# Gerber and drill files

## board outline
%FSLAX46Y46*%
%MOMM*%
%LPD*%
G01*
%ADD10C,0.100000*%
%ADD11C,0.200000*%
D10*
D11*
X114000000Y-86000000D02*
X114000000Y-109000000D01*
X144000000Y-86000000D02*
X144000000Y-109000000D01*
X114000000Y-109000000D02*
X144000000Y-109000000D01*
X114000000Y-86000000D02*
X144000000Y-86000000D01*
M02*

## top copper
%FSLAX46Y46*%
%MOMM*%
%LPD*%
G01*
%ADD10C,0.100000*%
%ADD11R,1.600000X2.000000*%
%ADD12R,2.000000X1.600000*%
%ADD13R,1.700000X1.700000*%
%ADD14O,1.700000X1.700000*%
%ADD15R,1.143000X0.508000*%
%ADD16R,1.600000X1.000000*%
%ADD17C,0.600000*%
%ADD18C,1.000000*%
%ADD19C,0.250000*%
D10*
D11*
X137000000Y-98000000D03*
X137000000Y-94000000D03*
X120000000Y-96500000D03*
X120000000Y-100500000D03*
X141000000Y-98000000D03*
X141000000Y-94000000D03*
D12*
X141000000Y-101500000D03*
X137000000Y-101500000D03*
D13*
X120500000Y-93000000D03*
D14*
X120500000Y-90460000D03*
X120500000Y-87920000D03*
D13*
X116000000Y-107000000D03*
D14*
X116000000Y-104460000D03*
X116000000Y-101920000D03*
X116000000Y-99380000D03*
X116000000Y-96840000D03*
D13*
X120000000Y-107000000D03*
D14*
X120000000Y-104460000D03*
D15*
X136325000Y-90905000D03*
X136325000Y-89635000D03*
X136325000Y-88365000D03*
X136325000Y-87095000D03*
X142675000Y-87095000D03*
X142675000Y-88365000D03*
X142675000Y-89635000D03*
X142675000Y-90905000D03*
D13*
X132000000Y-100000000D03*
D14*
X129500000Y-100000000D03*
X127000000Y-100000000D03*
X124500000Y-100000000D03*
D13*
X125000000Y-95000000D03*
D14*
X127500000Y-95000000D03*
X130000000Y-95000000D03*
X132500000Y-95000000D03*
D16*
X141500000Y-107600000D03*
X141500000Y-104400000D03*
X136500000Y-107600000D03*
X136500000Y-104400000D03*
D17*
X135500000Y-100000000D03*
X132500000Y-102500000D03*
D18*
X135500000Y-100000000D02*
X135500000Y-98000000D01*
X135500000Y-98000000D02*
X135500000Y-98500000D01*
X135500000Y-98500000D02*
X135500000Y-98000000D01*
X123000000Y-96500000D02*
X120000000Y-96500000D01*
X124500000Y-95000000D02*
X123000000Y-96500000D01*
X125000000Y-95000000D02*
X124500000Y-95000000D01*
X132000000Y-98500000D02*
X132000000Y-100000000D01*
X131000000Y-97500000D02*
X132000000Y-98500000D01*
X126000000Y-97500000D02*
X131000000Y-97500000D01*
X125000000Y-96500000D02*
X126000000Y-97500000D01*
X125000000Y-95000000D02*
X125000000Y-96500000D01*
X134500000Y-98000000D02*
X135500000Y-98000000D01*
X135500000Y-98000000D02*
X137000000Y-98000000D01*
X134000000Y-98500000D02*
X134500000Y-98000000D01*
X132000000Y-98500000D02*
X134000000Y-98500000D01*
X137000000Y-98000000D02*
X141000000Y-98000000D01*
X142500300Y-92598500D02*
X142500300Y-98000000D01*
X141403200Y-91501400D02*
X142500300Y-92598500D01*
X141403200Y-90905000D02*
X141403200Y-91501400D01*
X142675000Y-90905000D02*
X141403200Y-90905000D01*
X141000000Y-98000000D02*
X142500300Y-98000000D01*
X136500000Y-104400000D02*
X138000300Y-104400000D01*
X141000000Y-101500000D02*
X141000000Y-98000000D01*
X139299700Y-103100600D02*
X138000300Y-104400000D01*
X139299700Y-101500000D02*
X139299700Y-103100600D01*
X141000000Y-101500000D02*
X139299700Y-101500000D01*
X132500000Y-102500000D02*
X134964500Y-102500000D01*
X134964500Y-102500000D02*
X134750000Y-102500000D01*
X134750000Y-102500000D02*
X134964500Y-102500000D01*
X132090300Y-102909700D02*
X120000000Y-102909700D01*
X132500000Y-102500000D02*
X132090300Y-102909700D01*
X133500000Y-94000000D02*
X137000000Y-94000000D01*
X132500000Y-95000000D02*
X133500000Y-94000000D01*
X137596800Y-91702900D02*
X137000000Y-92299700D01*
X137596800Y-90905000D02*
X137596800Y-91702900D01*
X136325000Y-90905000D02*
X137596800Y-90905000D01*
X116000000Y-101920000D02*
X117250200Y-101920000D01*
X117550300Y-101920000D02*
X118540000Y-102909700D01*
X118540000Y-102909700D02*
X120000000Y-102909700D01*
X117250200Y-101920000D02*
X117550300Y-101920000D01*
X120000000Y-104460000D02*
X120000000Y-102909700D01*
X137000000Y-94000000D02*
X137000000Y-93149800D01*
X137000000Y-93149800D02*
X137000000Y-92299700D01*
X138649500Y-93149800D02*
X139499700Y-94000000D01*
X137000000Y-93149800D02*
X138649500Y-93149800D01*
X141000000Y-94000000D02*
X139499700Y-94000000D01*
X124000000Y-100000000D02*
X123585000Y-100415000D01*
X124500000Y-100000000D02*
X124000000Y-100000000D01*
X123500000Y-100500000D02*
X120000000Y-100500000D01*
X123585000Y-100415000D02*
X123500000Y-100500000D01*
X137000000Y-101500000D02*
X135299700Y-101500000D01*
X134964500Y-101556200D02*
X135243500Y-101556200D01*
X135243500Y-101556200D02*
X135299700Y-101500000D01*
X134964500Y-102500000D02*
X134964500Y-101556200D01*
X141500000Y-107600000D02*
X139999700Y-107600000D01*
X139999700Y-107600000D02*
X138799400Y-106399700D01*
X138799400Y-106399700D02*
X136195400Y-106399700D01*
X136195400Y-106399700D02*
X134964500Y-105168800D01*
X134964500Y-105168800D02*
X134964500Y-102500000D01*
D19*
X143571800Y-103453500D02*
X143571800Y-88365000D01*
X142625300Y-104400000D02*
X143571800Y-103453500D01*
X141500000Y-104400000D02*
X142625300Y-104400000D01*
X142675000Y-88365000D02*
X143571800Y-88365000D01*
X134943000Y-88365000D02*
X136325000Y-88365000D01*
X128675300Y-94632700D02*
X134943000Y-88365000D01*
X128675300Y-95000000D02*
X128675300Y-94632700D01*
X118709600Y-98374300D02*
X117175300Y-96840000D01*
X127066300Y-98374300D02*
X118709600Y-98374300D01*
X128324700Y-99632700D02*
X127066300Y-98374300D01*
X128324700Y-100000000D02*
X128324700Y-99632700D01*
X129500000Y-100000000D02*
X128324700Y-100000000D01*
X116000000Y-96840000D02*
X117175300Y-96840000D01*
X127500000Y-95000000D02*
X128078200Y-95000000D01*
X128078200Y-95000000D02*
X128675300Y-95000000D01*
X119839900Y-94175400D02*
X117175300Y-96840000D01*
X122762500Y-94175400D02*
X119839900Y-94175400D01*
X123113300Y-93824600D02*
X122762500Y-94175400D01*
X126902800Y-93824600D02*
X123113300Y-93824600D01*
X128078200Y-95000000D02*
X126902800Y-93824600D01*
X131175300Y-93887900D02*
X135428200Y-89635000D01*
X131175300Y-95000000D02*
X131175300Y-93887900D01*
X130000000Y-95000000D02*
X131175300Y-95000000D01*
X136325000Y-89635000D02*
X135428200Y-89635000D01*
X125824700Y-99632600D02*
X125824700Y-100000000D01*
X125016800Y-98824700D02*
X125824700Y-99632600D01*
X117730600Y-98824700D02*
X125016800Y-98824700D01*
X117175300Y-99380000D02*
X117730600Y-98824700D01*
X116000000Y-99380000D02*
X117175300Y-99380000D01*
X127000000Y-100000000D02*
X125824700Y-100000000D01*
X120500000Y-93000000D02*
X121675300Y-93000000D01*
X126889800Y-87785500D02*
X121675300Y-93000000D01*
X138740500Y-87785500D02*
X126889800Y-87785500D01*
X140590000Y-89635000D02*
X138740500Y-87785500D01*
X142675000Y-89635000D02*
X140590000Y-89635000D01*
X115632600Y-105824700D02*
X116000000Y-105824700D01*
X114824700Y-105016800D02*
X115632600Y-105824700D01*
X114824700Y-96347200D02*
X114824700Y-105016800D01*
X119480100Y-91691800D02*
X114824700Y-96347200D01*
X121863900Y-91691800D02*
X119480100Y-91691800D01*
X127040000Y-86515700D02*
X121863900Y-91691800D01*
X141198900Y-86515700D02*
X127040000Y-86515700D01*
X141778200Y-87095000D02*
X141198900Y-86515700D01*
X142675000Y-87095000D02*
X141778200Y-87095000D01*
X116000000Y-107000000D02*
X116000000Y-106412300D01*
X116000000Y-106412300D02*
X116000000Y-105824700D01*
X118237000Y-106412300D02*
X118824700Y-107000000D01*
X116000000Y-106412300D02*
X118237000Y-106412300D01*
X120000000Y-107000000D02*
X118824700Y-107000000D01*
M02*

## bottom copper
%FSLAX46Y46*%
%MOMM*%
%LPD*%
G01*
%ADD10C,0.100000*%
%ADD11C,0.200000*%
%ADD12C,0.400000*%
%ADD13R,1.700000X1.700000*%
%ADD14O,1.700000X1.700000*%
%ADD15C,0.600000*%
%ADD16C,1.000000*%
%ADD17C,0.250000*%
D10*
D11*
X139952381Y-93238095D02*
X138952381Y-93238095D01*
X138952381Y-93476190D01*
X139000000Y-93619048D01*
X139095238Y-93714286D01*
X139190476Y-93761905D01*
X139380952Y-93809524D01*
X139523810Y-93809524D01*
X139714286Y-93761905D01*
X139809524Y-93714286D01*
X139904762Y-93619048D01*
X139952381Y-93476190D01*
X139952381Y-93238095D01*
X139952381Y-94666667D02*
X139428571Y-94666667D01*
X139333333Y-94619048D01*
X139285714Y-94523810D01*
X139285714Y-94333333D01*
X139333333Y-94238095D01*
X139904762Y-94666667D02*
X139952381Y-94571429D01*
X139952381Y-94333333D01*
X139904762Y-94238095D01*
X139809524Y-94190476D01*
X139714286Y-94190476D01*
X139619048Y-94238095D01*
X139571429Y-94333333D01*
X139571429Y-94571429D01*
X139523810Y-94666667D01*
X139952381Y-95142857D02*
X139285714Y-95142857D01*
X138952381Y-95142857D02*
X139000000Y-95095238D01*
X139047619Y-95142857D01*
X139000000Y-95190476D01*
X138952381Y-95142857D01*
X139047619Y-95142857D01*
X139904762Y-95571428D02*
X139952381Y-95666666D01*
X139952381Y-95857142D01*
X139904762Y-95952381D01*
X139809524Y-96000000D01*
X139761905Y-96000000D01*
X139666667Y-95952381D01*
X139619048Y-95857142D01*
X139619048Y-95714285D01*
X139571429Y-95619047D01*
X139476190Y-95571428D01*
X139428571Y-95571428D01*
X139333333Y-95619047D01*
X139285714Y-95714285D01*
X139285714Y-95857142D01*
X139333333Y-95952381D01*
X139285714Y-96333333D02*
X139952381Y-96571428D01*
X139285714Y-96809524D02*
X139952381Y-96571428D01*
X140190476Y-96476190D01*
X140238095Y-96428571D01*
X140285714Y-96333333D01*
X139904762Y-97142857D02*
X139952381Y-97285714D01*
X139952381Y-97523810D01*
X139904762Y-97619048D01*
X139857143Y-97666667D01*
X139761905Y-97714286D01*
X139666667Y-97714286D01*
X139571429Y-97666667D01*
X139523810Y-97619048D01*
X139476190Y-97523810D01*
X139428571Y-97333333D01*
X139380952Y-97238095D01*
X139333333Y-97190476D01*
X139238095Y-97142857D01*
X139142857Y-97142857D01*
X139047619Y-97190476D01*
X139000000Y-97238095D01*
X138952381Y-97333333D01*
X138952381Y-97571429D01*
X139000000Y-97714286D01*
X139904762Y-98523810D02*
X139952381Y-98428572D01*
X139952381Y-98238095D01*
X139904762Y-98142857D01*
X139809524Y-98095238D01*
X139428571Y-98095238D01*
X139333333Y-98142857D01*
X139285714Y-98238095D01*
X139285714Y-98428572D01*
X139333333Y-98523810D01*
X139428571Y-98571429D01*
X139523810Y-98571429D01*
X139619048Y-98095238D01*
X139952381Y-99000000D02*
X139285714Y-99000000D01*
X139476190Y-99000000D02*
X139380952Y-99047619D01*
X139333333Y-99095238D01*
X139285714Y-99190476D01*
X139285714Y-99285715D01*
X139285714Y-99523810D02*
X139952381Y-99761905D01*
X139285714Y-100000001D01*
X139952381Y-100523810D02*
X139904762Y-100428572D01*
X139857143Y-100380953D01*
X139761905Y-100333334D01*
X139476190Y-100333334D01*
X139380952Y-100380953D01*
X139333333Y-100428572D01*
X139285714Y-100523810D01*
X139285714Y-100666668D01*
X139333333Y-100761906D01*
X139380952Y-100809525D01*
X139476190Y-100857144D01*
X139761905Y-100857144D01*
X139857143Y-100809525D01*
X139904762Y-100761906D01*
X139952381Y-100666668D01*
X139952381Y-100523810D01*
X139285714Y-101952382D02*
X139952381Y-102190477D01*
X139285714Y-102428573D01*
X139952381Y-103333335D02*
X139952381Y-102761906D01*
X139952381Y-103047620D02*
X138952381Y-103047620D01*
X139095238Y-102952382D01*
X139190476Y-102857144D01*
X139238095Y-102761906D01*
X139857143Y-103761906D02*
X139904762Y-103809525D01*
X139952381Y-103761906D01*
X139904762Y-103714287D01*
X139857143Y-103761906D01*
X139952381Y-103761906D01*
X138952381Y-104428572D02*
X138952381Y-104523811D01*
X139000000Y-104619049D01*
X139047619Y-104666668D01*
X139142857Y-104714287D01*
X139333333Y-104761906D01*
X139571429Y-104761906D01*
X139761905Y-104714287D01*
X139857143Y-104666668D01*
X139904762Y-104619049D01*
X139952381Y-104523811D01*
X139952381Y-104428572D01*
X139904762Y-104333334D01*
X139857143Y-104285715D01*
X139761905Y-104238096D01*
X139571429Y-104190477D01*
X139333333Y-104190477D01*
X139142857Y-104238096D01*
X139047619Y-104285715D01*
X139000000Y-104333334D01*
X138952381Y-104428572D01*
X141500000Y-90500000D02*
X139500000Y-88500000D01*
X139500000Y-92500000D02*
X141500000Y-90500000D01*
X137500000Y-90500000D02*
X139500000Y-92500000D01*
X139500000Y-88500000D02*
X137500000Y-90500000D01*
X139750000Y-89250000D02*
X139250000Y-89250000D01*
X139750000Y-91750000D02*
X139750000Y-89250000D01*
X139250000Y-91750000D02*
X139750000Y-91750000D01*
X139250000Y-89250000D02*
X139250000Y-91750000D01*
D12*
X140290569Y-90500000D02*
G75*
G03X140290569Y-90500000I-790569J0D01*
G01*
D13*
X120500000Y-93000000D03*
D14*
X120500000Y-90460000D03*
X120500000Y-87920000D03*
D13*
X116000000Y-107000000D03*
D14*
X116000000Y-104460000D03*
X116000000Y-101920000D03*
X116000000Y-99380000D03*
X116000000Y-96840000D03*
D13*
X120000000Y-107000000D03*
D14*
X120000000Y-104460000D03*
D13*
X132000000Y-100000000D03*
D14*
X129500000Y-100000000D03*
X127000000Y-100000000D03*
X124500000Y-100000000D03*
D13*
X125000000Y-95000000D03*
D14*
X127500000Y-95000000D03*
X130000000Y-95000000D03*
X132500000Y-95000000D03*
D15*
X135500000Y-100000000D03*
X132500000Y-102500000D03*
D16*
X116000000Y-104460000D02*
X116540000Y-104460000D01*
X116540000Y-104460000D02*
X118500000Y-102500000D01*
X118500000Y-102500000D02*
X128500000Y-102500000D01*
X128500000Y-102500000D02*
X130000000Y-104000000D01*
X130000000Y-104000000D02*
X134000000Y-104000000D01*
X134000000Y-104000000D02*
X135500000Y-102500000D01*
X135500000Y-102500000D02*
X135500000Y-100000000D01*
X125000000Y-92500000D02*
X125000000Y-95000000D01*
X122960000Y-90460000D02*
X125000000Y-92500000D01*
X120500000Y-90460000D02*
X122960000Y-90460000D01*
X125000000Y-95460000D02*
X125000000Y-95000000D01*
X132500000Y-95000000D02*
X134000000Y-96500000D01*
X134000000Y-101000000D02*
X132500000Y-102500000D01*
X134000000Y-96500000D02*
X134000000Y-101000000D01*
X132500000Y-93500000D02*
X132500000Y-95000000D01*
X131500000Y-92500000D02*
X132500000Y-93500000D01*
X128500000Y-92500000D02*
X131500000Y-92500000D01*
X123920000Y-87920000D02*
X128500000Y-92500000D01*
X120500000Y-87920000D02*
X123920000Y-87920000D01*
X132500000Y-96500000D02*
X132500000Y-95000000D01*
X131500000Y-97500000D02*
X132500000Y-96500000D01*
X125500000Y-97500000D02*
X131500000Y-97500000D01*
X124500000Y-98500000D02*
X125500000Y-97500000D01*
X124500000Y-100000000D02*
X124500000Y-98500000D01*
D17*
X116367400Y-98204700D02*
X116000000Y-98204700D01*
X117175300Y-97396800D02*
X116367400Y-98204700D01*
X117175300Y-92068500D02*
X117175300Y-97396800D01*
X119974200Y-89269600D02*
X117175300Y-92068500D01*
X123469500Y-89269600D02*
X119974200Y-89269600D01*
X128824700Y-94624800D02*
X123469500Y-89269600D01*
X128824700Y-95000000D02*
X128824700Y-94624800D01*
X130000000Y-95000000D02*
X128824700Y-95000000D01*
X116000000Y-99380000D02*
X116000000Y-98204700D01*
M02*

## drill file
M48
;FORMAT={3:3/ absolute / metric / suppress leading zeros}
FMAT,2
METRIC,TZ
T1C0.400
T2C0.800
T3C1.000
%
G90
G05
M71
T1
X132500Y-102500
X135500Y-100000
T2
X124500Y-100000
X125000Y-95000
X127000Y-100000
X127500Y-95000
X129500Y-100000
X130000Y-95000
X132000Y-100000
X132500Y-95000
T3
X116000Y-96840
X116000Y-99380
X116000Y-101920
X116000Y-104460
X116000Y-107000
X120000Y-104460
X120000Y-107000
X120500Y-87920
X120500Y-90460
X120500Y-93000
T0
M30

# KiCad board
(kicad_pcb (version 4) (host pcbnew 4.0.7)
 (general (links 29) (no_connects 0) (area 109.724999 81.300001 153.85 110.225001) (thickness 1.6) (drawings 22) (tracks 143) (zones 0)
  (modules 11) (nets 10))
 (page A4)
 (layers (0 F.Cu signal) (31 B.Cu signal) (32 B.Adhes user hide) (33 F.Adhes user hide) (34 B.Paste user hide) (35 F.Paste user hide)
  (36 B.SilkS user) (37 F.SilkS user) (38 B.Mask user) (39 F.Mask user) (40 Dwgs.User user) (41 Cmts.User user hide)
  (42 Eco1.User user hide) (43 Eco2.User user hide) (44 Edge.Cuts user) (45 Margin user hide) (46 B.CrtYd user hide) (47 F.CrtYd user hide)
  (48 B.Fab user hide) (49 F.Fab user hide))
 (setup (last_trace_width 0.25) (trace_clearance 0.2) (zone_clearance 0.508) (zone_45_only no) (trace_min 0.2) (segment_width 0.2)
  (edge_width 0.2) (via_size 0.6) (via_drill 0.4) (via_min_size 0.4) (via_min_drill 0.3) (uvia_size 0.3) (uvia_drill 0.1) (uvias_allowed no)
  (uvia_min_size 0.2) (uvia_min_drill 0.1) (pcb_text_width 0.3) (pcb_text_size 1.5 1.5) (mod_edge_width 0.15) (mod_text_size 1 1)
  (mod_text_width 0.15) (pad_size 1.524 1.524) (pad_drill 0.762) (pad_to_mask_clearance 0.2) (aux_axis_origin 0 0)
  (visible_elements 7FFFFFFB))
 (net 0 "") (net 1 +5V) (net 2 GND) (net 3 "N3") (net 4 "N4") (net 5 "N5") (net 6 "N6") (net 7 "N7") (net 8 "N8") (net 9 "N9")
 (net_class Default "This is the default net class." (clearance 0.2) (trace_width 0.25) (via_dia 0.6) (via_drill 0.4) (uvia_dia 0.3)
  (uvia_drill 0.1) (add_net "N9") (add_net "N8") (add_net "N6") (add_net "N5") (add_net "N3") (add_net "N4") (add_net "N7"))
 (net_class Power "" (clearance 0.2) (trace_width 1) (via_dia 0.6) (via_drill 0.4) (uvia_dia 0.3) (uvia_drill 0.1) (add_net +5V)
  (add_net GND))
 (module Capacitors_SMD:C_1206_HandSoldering (layer F.Cu) (at 137 96 90)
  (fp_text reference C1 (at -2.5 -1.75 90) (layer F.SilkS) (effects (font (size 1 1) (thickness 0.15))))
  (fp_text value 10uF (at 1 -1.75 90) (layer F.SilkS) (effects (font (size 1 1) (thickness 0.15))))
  (pad 1 smd rect (at -2 0 90) (size 2 1.6) (layers F.Cu F.Paste F.Mask) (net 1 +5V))
  (pad 2 smd rect (at 2 0 90) (size 2 1.6) (layers F.Cu F.Paste F.Mask) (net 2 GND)))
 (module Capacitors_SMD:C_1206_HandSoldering (layer F.Cu) (at 120 98.5 270)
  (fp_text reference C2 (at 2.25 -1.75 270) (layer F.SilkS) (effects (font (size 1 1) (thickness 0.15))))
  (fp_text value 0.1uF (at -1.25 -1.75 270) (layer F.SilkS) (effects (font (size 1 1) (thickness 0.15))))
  (pad 1 smd rect (at -2 0 270) (size 2 1.6) (layers F.Cu F.Paste F.Mask) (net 1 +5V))
  (pad 2 smd rect (at 2 0 270) (size 2 1.6) (layers F.Cu F.Paste F.Mask) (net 2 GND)))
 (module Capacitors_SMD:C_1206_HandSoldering (layer F.Cu) (at 141 96 90)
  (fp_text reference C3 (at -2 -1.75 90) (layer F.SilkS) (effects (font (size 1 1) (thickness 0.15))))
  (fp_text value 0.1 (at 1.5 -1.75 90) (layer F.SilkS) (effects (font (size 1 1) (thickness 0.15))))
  (pad 1 smd rect (at -2 0 90) (size 2 1.6) (layers F.Cu F.Paste F.Mask) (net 1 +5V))
  (pad 2 smd rect (at 2 0 90) (size 2 1.6) (layers F.Cu F.Paste F.Mask) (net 2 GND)))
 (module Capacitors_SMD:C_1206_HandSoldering (layer F.Cu) (at 139 101.5 180)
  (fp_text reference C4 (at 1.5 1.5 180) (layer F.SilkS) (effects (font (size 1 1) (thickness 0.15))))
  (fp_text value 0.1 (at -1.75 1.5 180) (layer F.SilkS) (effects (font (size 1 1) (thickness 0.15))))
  (pad 1 smd rect (at -2 0 180) (size 2 1.6) (layers F.Cu F.Paste F.Mask) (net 1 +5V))
  (pad 2 smd rect (at 2 0 180) (size 2 1.6) (layers F.Cu F.Paste F.Mask) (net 2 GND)))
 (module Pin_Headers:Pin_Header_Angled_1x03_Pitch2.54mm (layer F.Cu) (at 120.5 93 180)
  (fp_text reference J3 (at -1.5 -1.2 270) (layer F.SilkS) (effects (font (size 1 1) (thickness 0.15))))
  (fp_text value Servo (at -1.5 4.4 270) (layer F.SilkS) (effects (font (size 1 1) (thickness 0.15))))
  (pad 1 thru_hole rect (at 0 0 180) (size 1.7 1.7) (drill 1) (layers *.Cu *.Mask) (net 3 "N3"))
  (pad 2 thru_hole oval (at 0 2.54 180) (size 1.7 1.7) (drill 1) (layers *.Cu *.Mask) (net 1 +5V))
  (pad 3 thru_hole oval (at 0 5.08 180) (size 1.7 1.7) (drill 1) (layers *.Cu *.Mask) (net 2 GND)))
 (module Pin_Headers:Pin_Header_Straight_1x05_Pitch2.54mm (layer F.Cu) (at 116 107 180)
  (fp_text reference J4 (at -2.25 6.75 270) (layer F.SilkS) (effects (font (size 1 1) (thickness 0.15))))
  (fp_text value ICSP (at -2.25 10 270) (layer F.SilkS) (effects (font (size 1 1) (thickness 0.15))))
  (pad 1 thru_hole rect (at 0 0 180) (size 1.7 1.7) (drill 1) (layers *.Cu *.Mask) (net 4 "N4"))
  (pad 2 thru_hole oval (at 0 2.54 180) (size 1.7 1.7) (drill 1) (layers *.Cu *.Mask) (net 1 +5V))
  (pad 3 thru_hole oval (at 0 5.08 180) (size 1.7 1.7) (drill 1) (layers *.Cu *.Mask) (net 2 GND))
  (pad 4 thru_hole oval (at 0 7.62 180) (size 1.7 1.7) (drill 1) (layers *.Cu *.Mask) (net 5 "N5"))
  (pad 5 thru_hole oval (at 0 10.16 180) (size 1.7 1.7) (drill 1) (layers *.Cu *.Mask) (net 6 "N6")))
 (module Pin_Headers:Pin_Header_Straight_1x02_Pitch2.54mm (layer F.Cu) (at 120 107 180)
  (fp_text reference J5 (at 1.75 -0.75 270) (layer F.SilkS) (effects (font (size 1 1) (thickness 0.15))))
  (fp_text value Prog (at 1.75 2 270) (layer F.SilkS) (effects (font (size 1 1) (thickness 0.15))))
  (pad 1 thru_hole rect (at 0 0 180) (size 1.7 1.7) (drill 1) (layers *.Cu *.Mask) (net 4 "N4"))
  (pad 2 thru_hole oval (at 0 2.54 180) (size 1.7 1.7) (drill 1) (layers *.Cu *.Mask) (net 2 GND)))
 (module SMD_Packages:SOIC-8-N (layer F.Cu) (at 139.5 89 90)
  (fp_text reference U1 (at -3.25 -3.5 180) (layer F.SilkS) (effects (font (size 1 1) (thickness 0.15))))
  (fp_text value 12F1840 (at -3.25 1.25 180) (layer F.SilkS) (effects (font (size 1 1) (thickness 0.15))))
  (pad 8 smd rect (at -1.905 -3.175 90) (size 0.508 1.143) (layers F.Cu F.Paste F.Mask) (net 2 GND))
  (pad 7 smd rect (at -0.635 -3.175 90) (size 0.508 1.143) (layers F.Cu F.Paste F.Mask) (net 5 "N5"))
  (pad 6 smd rect (at 0.635 -3.175 90) (size 0.508 1.143) (layers F.Cu F.Paste F.Mask) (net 6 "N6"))
  (pad 5 smd rect (at 1.905 -3.175 90) (size 0.508 1.143) (layers F.Cu F.Paste F.Mask) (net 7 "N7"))
  (pad 4 smd rect (at 1.905 3.175 90) (size 0.508 1.143) (layers F.Cu F.Paste F.Mask) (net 4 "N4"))
  (pad 3 smd rect (at 0.635 3.175 90) (size 0.508 1.143) (layers F.Cu F.Paste F.Mask) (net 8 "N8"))
  (pad 2 smd rect (at -0.635 3.175 90) (size 0.508 1.143) (layers F.Cu F.Paste F.Mask) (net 3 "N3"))
  (pad 1 smd rect (at -1.905 3.175 90) (size 0.508 1.143) (layers F.Cu F.Paste F.Mask) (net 1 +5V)))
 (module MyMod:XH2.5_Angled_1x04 (layer F.Cu) (at 132 100 270)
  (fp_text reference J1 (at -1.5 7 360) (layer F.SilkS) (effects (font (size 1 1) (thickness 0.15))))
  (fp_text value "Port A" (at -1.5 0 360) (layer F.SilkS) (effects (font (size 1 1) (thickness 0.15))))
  (pad 1 thru_hole rect (at 0 0 270) (size 1.7 1.7) (drill 0.8) (layers *.Cu *.Mask) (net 1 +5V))
  (pad 2 thru_hole oval (at 0 2.5 270) (size 1.7 1.7) (drill 0.8) (layers *.Cu *.Mask) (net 6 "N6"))
  (pad 3 thru_hole oval (at 0 5 270) (size 1.7 1.7) (drill 0.8) (layers *.Cu *.Mask) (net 5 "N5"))
  (pad 4 thru_hole oval (at 0 7.5 270) (size 1.7 1.7) (drill 0.8) (layers *.Cu *.Mask) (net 2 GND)))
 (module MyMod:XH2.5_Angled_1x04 (layer F.Cu) (at 125 95 90)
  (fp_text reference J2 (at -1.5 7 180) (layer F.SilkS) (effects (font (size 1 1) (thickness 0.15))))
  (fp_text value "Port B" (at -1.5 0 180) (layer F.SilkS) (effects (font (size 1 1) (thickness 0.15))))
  (pad 1 thru_hole rect (at 0 0 90) (size 1.7 1.7) (drill 0.8) (layers *.Cu *.Mask) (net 1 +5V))
  (pad 2 thru_hole oval (at 0 2.5 90) (size 1.7 1.7) (drill 0.8) (layers *.Cu *.Mask) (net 6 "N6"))
  (pad 3 thru_hole oval (at 0 5 90) (size 1.7 1.7) (drill 0.8) (layers *.Cu *.Mask) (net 5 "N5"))
  (pad 4 thru_hole oval (at 0 7.5 90) (size 1.7 1.7) (drill 0.8) (layers *.Cu *.Mask) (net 2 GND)))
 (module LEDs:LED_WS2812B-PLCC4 (layer F.Cu) (at 139 106)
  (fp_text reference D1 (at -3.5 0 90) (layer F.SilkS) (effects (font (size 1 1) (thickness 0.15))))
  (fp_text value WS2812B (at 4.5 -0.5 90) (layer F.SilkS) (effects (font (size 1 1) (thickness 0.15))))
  (pad 3 smd rect (at 2.5 1.6) (size 1.6 1) (layers F.Cu F.Paste F.Mask) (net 2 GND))
  (pad 4 smd rect (at 2.5 -1.6) (size 1.6 1) (layers F.Cu F.Paste F.Mask) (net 8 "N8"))
  (pad 2 smd rect (at -2.5 1.6) (size 1.6 1) (layers F.Cu F.Paste F.Mask) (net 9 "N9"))
  (pad 1 smd rect (at -2.5 -1.6) (size 1.6 1) (layers F.Cu F.Paste F.Mask) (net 1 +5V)))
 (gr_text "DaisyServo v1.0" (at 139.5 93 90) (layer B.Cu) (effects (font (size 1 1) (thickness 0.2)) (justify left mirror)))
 (gr_line (start 141.5 90.5) (end 139.5 88.5) (angle 90) (layer B.Cu) (width 0.2))
 (gr_line (start 139.5 92.5) (end 141.5 90.5) (angle 90) (layer B.Cu) (width 0.2))
 (gr_line (start 137.5 90.5) (end 139.5 92.5) (angle 90) (layer B.Cu) (width 0.2))
 (gr_line (start 139.5 88.5) (end 137.5 90.5) (angle 90) (layer B.Cu) (width 0.2))
 (gr_line (start 139.75 89.25) (end 139.25 89.25) (angle 90) (layer B.Cu) (width 0.2))
 (gr_line (start 139.75 91.75) (end 139.75 89.25) (angle 90) (layer B.Cu) (width 0.2))
 (gr_line (start 139.25 91.75) (end 139.75 91.75) (angle 90) (layer B.Cu) (width 0.2))
 (gr_line (start 139.25 89.25) (end 139.25 91.75) (angle 90) (layer B.Cu) (width 0.2))
 (gr_circle (center 139.5 90.5) (end 139.75 89.75) (layer B.Cu) (width 0.4))
 (gr_line (start 114 86) (end 114 109) (angle 90) (layer Edge.Cuts) (width 0.2))
 (gr_line (start 144 86) (end 144 109) (angle 90) (layer Edge.Cuts) (width 0.2))
 (gr_line (start 114 109) (end 144 109) (angle 90) (layer Edge.Cuts) (width 0.2))
 (gr_line (start 114 86) (end 144 86) (angle 90) (layer Edge.Cuts) (width 0.2))
 (segment (start 116 104.46) (end 116.54 104.46) (width 1) (layer B.Cu) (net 1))
 (segment (start 116.54 104.46) (end 118.5 102.5) (width 1) (layer B.Cu) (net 1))
 (segment (start 118.5 102.5) (end 128.5 102.5) (width 1) (layer B.Cu) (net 1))
 (segment (start 128.5 102.5) (end 130 104) (width 1) (layer B.Cu) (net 1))
 (segment (start 130 104) (end 134 104) (width 1) (layer B.Cu) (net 1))
 (segment (start 134 104) (end 135.5 102.5) (width 1) (layer B.Cu) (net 1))
 (segment (start 135.5 102.5) (end 135.5 100) (width 1) (layer B.Cu) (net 1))
 (via (at 135.5 100) (size 0.6) (drill 0.4) (layers F.Cu B.Cu) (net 1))
 (segment (start 135.5 100) (end 135.5 98) (width 1) (layer F.Cu) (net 1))
 (segment (start 135.5 98) (end 135.5 98.5) (width 1) (layer F.Cu) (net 1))
 (segment (start 135.5 98.5) (end 135.5 98) (width 1) (layer F.Cu) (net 1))
 (segment (start 123 96.5) (end 120 96.5) (width 1) (layer F.Cu) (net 1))
 (segment (start 124.5 95) (end 123 96.5) (width 1) (layer F.Cu) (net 1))
 (segment (start 125 95) (end 124.5 95) (width 1) (layer F.Cu) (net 1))
 (segment (start 125 92.5) (end 125 95) (width 1) (layer B.Cu) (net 1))
 (segment (start 122.96 90.46) (end 125 92.5) (width 1) (layer B.Cu) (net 1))
 (segment (start 120.5 90.46) (end 122.96 90.46) (width 1) (layer B.Cu) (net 1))
 (segment (start 132 98.5) (end 132 100) (width 1) (layer F.Cu) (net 1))
 (segment (start 131 97.5) (end 132 98.5) (width 1) (layer F.Cu) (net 1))
 (segment (start 126 97.5) (end 131 97.5) (width 1) (layer F.Cu) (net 1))
 (segment (start 125 96.5) (end 126 97.5) (width 1) (layer F.Cu) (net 1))
 (segment (start 125 95) (end 125 96.5) (width 1) (layer F.Cu) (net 1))
 (segment (start 134.5 98) (end 135.5 98) (width 1) (layer F.Cu) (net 1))
 (segment (start 135.5 98) (end 137 98) (width 1) (layer F.Cu) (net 1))
 (segment (start 134 98.5) (end 134.5 98) (width 1) (layer F.Cu) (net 1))
 (segment (start 132 98.5) (end 134 98.5) (width 1) (layer F.Cu) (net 1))
 (segment (start 137 98) (end 141 98) (width 1) (layer F.Cu) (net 1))
 (segment (start 142.5003 92.5985) (end 142.5003 98) (width 1) (layer F.Cu) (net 1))
 (segment (start 141.4032 91.5014) (end 142.5003 92.5985) (width 1) (layer F.Cu) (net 1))
 (segment (start 141.4032 90.905) (end 141.4032 91.5014) (width 1) (layer F.Cu) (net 1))
 (segment (start 142.675 90.905) (end 141.4032 90.905) (width 1) (layer F.Cu) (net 1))
 (segment (start 141 98) (end 142.5003 98) (width 1) (layer F.Cu) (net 1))
 (segment (start 125 95.46) (end 125 95) (width 1) (layer B.Cu) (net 1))
 (segment (start 136.5 104.4) (end 138.0003 104.4) (width 1) (layer F.Cu) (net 1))
 (segment (start 141 101.5) (end 141 98) (width 1) (layer F.Cu) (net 1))
 (segment (start 139.2997 103.1006) (end 138.0003 104.4) (width 1) (layer F.Cu) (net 1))
 (segment (start 139.2997 101.5) (end 139.2997 103.1006) (width 1) (layer F.Cu) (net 1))
 (segment (start 141 101.5) (end 139.2997 101.5) (width 1) (layer F.Cu) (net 1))
 (segment (start 132.5 102.5) (end 134.9645 102.5) (width 1) (layer F.Cu) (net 2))
 (segment (start 134.9645 102.5) (end 134.75 102.5) (width 1) (layer F.Cu) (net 2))
 (segment (start 134.75 102.5) (end 134.9645 102.5) (width 1) (layer F.Cu) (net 2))
 (segment (start 132.5 95) (end 134 96.5) (width 1) (layer B.Cu) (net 2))
 (segment (start 132.0903 102.9097) (end 120 102.9097) (width 1) (layer F.Cu) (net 2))
 (segment (start 132.5 102.5) (end 132.0903 102.9097) (width 1) (layer F.Cu) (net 2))
 (via (at 132.5 102.5) (size 0.6) (drill 0.4) (layers F.Cu B.Cu) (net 2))
 (segment (start 134 101) (end 132.5 102.5) (width 1) (layer B.Cu) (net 2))
 (segment (start 134 96.5) (end 134 101) (width 1) (layer B.Cu) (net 2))
 (segment (start 132.5 93.5) (end 132.5 95) (width 1) (layer B.Cu) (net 2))
 (segment (start 131.5 92.5) (end 132.5 93.5) (width 1) (layer B.Cu) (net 2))
 (segment (start 128.5 92.5) (end 131.5 92.5) (width 1) (layer B.Cu) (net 2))
 (segment (start 123.92 87.92) (end 128.5 92.5) (width 1) (layer B.Cu) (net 2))
 (segment (start 120.5 87.92) (end 123.92 87.92) (width 1) (layer B.Cu) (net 2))
 (segment (start 132.5 96.5) (end 132.5 95) (width 1) (layer B.Cu) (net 2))
 (segment (start 131.5 97.5) (end 132.5 96.5) (width 1) (layer B.Cu) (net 2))
 (segment (start 125.5 97.5) (end 131.5 97.5) (width 1) (layer B.Cu) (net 2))
 (segment (start 124.5 98.5) (end 125.5 97.5) (width 1) (layer B.Cu) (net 2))
 (segment (start 124.5 100) (end 124.5 98.5) (width 1) (layer B.Cu) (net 2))
 (segment (start 133.5 94) (end 137 94) (width 1) (layer F.Cu) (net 2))
 (segment (start 132.5 95) (end 133.5 94) (width 1) (layer F.Cu) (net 2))
 (segment (start 137.5968 91.7029) (end 137 92.2997) (width 1) (layer F.Cu) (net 2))
 (segment (start 137.5968 90.905) (end 137.5968 91.7029) (width 1) (layer F.Cu) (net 2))
 (segment (start 136.325 90.905) (end 137.5968 90.905) (width 1) (layer F.Cu) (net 2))
 (segment (start 116 101.92) (end 117.2502 101.92) (width 1) (layer F.Cu) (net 2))
 (segment (start 117.5503 101.92) (end 118.54 102.9097) (width 1) (layer F.Cu) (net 2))
 (segment (start 118.54 102.9097) (end 120 102.9097) (width 1) (layer F.Cu) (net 2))
 (segment (start 117.2502 101.92) (end 117.5503 101.92) (width 1) (layer F.Cu) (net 2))
 (segment (start 120 104.46) (end 120 102.9097) (width 1) (layer F.Cu) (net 2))
 (segment (start 137 94) (end 137 93.1498) (width 1) (layer F.Cu) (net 2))
 (segment (start 137 93.1498) (end 137 92.2997) (width 1) (layer F.Cu) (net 2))
 (segment (start 138.6495 93.1498) (end 139.4997 94) (width 1) (layer F.Cu) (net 2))
 (segment (start 137 93.1498) (end 138.6495 93.1498) (width 1) (layer F.Cu) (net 2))
 (segment (start 141 94) (end 139.4997 94) (width 1) (layer F.Cu) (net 2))
 (segment (start 124 100) (end 123.585 100.415) (width 1) (layer F.Cu) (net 2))
 (segment (start 124.5 100) (end 124 100) (width 1) (layer F.Cu) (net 2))
 (segment (start 123.5 100.5) (end 120 100.5) (width 1) (layer F.Cu) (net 2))
 (segment (start 123.585 100.415) (end 123.5 100.5) (width 1) (layer F.Cu) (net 2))
 (segment (start 137 101.5) (end 135.2997 101.5) (width 1) (layer F.Cu) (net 2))
 (segment (start 134.9645 101.5562) (end 135.2435 101.5562) (width 1) (layer F.Cu) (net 2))
 (segment (start 135.2435 101.5562) (end 135.2997 101.5) (width 1) (layer F.Cu) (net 2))
 (segment (start 134.9645 102.5) (end 134.9645 101.5562) (width 1) (layer F.Cu) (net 2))
 (segment (start 141.5 107.6) (end 139.9997 107.6) (width 1) (layer F.Cu) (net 2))
 (segment (start 139.9997 107.6) (end 138.7994 106.3997) (width 1) (layer F.Cu) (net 2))
 (segment (start 138.7994 106.3997) (end 136.1954 106.3997) (width 1) (layer F.Cu) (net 2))
 (segment (start 136.1954 106.3997) (end 134.9645 105.1688) (width 1) (layer F.Cu) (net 2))
 (segment (start 134.9645 105.1688) (end 134.9645 102.5) (width 1) (layer F.Cu) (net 2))
 (segment (start 143.5718 103.4535) (end 143.5718 88.365) (width 0.25) (layer F.Cu) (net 8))
 (segment (start 142.6253 104.4) (end 143.5718 103.4535) (width 0.25) (layer F.Cu) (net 8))
 (segment (start 141.5 104.4) (end 142.6253 104.4) (width 0.25) (layer F.Cu) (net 8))
 (segment (start 142.675 88.365) (end 143.5718 88.365) (width 0.25) (layer F.Cu) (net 8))
 (segment (start 134.943 88.365) (end 136.325 88.365) (width 0.25) (layer F.Cu) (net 6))
 (segment (start 128.6753 94.6327) (end 134.943 88.365) (width 0.25) (layer F.Cu) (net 6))
 (segment (start 128.6753 95) (end 128.6753 94.6327) (width 0.25) (layer F.Cu) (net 6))
 (segment (start 118.7096 98.3743) (end 117.1753 96.84) (width 0.25) (layer F.Cu) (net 6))
 (segment (start 127.0663 98.3743) (end 118.7096 98.3743) (width 0.25) (layer F.Cu) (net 6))
 (segment (start 128.3247 99.6327) (end 127.0663 98.3743) (width 0.25) (layer F.Cu) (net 6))
 (segment (start 128.3247 100) (end 128.3247 99.6327) (width 0.25) (layer F.Cu) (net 6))
 (segment (start 129.5 100) (end 128.3247 100) (width 0.25) (layer F.Cu) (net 6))
 (segment (start 116 96.84) (end 117.1753 96.84) (width 0.25) (layer F.Cu) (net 6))
 (segment (start 127.5 95) (end 128.0782 95) (width 0.25) (layer F.Cu) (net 6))
 (segment (start 128.0782 95) (end 128.6753 95) (width 0.25) (layer F.Cu) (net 6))
 (segment (start 119.8399 94.1754) (end 117.1753 96.84) (width 0.25) (layer F.Cu) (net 6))
 (segment (start 122.7625 94.1754) (end 119.8399 94.1754) (width 0.25) (layer F.Cu) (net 6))
 (segment (start 123.1133 93.8246) (end 122.7625 94.1754) (width 0.25) (layer F.Cu) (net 6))
 (segment (start 126.9028 93.8246) (end 123.1133 93.8246) (width 0.25) (layer F.Cu) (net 6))
 (segment (start 128.0782 95) (end 126.9028 93.8246) (width 0.25) (layer F.Cu) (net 6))
 (segment (start 131.1753 93.8879) (end 135.4282 89.635) (width 0.25) (layer F.Cu) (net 5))
 (segment (start 131.1753 95) (end 131.1753 93.8879) (width 0.25) (layer F.Cu) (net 5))
 (segment (start 130 95) (end 131.1753 95) (width 0.25) (layer F.Cu) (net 5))
 (segment (start 136.325 89.635) (end 135.4282 89.635) (width 0.25) (layer F.Cu) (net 5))
 (segment (start 116.3674 98.2047) (end 116 98.2047) (width 0.25) (layer B.Cu) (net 5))
 (segment (start 117.1753 97.3968) (end 116.3674 98.2047) (width 0.25) (layer B.Cu) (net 5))
 (segment (start 117.1753 92.0685) (end 117.1753 97.3968) (width 0.25) (layer B.Cu) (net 5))
 (segment (start 119.9742 89.2696) (end 117.1753 92.0685) (width 0.25) (layer B.Cu) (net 5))
 (segment (start 123.4695 89.2696) (end 119.9742 89.2696) (width 0.25) (layer B.Cu) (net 5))
 (segment (start 128.8247 94.6248) (end 123.4695 89.2696) (width 0.25) (layer B.Cu) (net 5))
 (segment (start 128.8247 95) (end 128.8247 94.6248) (width 0.25) (layer B.Cu) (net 5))
 (segment (start 130 95) (end 128.8247 95) (width 0.25) (layer B.Cu) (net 5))
 (segment (start 116 99.38) (end 116 98.2047) (width 0.25) (layer B.Cu) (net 5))
 (segment (start 125.8247 99.6326) (end 125.8247 100) (width 0.25) (layer F.Cu) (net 5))
 (segment (start 125.0168 98.8247) (end 125.8247 99.6326) (width 0.25) (layer F.Cu) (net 5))
 (segment (start 117.7306 98.8247) (end 125.0168 98.8247) (width 0.25) (layer F.Cu) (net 5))
 (segment (start 117.1753 99.38) (end 117.7306 98.8247) (width 0.25) (layer F.Cu) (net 5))
 (segment (start 116 99.38) (end 117.1753 99.38) (width 0.25) (layer F.Cu) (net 5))
 (segment (start 127 100) (end 125.8247 100) (width 0.25) (layer F.Cu) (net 5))
 (segment (start 120.5 93) (end 121.6753 93) (width 0.25) (layer F.Cu) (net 3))
 (segment (start 126.8898 87.7855) (end 121.6753 93) (width 0.25) (layer F.Cu) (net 3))
 (segment (start 138.7405 87.7855) (end 126.8898 87.7855) (width 0.25) (layer F.Cu) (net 3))
 (segment (start 140.59 89.635) (end 138.7405 87.7855) (width 0.25) (layer F.Cu) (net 3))
 (segment (start 142.675 89.635) (end 140.59 89.635) (width 0.25) (layer F.Cu) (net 3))
 (segment (start 115.6326 105.8247) (end 116 105.8247) (width 0.25) (layer F.Cu) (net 4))
 (segment (start 114.8247 105.0168) (end 115.6326 105.8247) (width 0.25) (layer F.Cu) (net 4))
 (segment (start 114.8247 96.3472) (end 114.8247 105.0168) (width 0.25) (layer F.Cu) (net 4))
 (segment (start 119.4801 91.6918) (end 114.8247 96.3472) (width 0.25) (layer F.Cu) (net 4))
 (segment (start 121.8639 91.6918) (end 119.4801 91.6918) (width 0.25) (layer F.Cu) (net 4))
 (segment (start 127.04 86.5157) (end 121.8639 91.6918) (width 0.25) (layer F.Cu) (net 4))
 (segment (start 141.1989 86.5157) (end 127.04 86.5157) (width 0.25) (layer F.Cu) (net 4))
 (segment (start 141.7782 87.095) (end 141.1989 86.5157) (width 0.25) (layer F.Cu) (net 4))
 (segment (start 142.675 87.095) (end 141.7782 87.095) (width 0.25) (layer F.Cu) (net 4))
 (segment (start 116 107) (end 116 106.4123) (width 0.25) (layer F.Cu) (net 4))
 (segment (start 116 106.4123) (end 116 105.8247) (width 0.25) (layer F.Cu) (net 4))
 (segment (start 118.237 106.4123) (end 118.8247 107) (width 0.25) (layer F.Cu) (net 4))
 (segment (start 116 106.4123) (end 118.237 106.4123) (width 0.25) (layer F.Cu) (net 4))
 (segment (start 120 107) (end 118.8247 107) (width 0.25) (layer F.Cu) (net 4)))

